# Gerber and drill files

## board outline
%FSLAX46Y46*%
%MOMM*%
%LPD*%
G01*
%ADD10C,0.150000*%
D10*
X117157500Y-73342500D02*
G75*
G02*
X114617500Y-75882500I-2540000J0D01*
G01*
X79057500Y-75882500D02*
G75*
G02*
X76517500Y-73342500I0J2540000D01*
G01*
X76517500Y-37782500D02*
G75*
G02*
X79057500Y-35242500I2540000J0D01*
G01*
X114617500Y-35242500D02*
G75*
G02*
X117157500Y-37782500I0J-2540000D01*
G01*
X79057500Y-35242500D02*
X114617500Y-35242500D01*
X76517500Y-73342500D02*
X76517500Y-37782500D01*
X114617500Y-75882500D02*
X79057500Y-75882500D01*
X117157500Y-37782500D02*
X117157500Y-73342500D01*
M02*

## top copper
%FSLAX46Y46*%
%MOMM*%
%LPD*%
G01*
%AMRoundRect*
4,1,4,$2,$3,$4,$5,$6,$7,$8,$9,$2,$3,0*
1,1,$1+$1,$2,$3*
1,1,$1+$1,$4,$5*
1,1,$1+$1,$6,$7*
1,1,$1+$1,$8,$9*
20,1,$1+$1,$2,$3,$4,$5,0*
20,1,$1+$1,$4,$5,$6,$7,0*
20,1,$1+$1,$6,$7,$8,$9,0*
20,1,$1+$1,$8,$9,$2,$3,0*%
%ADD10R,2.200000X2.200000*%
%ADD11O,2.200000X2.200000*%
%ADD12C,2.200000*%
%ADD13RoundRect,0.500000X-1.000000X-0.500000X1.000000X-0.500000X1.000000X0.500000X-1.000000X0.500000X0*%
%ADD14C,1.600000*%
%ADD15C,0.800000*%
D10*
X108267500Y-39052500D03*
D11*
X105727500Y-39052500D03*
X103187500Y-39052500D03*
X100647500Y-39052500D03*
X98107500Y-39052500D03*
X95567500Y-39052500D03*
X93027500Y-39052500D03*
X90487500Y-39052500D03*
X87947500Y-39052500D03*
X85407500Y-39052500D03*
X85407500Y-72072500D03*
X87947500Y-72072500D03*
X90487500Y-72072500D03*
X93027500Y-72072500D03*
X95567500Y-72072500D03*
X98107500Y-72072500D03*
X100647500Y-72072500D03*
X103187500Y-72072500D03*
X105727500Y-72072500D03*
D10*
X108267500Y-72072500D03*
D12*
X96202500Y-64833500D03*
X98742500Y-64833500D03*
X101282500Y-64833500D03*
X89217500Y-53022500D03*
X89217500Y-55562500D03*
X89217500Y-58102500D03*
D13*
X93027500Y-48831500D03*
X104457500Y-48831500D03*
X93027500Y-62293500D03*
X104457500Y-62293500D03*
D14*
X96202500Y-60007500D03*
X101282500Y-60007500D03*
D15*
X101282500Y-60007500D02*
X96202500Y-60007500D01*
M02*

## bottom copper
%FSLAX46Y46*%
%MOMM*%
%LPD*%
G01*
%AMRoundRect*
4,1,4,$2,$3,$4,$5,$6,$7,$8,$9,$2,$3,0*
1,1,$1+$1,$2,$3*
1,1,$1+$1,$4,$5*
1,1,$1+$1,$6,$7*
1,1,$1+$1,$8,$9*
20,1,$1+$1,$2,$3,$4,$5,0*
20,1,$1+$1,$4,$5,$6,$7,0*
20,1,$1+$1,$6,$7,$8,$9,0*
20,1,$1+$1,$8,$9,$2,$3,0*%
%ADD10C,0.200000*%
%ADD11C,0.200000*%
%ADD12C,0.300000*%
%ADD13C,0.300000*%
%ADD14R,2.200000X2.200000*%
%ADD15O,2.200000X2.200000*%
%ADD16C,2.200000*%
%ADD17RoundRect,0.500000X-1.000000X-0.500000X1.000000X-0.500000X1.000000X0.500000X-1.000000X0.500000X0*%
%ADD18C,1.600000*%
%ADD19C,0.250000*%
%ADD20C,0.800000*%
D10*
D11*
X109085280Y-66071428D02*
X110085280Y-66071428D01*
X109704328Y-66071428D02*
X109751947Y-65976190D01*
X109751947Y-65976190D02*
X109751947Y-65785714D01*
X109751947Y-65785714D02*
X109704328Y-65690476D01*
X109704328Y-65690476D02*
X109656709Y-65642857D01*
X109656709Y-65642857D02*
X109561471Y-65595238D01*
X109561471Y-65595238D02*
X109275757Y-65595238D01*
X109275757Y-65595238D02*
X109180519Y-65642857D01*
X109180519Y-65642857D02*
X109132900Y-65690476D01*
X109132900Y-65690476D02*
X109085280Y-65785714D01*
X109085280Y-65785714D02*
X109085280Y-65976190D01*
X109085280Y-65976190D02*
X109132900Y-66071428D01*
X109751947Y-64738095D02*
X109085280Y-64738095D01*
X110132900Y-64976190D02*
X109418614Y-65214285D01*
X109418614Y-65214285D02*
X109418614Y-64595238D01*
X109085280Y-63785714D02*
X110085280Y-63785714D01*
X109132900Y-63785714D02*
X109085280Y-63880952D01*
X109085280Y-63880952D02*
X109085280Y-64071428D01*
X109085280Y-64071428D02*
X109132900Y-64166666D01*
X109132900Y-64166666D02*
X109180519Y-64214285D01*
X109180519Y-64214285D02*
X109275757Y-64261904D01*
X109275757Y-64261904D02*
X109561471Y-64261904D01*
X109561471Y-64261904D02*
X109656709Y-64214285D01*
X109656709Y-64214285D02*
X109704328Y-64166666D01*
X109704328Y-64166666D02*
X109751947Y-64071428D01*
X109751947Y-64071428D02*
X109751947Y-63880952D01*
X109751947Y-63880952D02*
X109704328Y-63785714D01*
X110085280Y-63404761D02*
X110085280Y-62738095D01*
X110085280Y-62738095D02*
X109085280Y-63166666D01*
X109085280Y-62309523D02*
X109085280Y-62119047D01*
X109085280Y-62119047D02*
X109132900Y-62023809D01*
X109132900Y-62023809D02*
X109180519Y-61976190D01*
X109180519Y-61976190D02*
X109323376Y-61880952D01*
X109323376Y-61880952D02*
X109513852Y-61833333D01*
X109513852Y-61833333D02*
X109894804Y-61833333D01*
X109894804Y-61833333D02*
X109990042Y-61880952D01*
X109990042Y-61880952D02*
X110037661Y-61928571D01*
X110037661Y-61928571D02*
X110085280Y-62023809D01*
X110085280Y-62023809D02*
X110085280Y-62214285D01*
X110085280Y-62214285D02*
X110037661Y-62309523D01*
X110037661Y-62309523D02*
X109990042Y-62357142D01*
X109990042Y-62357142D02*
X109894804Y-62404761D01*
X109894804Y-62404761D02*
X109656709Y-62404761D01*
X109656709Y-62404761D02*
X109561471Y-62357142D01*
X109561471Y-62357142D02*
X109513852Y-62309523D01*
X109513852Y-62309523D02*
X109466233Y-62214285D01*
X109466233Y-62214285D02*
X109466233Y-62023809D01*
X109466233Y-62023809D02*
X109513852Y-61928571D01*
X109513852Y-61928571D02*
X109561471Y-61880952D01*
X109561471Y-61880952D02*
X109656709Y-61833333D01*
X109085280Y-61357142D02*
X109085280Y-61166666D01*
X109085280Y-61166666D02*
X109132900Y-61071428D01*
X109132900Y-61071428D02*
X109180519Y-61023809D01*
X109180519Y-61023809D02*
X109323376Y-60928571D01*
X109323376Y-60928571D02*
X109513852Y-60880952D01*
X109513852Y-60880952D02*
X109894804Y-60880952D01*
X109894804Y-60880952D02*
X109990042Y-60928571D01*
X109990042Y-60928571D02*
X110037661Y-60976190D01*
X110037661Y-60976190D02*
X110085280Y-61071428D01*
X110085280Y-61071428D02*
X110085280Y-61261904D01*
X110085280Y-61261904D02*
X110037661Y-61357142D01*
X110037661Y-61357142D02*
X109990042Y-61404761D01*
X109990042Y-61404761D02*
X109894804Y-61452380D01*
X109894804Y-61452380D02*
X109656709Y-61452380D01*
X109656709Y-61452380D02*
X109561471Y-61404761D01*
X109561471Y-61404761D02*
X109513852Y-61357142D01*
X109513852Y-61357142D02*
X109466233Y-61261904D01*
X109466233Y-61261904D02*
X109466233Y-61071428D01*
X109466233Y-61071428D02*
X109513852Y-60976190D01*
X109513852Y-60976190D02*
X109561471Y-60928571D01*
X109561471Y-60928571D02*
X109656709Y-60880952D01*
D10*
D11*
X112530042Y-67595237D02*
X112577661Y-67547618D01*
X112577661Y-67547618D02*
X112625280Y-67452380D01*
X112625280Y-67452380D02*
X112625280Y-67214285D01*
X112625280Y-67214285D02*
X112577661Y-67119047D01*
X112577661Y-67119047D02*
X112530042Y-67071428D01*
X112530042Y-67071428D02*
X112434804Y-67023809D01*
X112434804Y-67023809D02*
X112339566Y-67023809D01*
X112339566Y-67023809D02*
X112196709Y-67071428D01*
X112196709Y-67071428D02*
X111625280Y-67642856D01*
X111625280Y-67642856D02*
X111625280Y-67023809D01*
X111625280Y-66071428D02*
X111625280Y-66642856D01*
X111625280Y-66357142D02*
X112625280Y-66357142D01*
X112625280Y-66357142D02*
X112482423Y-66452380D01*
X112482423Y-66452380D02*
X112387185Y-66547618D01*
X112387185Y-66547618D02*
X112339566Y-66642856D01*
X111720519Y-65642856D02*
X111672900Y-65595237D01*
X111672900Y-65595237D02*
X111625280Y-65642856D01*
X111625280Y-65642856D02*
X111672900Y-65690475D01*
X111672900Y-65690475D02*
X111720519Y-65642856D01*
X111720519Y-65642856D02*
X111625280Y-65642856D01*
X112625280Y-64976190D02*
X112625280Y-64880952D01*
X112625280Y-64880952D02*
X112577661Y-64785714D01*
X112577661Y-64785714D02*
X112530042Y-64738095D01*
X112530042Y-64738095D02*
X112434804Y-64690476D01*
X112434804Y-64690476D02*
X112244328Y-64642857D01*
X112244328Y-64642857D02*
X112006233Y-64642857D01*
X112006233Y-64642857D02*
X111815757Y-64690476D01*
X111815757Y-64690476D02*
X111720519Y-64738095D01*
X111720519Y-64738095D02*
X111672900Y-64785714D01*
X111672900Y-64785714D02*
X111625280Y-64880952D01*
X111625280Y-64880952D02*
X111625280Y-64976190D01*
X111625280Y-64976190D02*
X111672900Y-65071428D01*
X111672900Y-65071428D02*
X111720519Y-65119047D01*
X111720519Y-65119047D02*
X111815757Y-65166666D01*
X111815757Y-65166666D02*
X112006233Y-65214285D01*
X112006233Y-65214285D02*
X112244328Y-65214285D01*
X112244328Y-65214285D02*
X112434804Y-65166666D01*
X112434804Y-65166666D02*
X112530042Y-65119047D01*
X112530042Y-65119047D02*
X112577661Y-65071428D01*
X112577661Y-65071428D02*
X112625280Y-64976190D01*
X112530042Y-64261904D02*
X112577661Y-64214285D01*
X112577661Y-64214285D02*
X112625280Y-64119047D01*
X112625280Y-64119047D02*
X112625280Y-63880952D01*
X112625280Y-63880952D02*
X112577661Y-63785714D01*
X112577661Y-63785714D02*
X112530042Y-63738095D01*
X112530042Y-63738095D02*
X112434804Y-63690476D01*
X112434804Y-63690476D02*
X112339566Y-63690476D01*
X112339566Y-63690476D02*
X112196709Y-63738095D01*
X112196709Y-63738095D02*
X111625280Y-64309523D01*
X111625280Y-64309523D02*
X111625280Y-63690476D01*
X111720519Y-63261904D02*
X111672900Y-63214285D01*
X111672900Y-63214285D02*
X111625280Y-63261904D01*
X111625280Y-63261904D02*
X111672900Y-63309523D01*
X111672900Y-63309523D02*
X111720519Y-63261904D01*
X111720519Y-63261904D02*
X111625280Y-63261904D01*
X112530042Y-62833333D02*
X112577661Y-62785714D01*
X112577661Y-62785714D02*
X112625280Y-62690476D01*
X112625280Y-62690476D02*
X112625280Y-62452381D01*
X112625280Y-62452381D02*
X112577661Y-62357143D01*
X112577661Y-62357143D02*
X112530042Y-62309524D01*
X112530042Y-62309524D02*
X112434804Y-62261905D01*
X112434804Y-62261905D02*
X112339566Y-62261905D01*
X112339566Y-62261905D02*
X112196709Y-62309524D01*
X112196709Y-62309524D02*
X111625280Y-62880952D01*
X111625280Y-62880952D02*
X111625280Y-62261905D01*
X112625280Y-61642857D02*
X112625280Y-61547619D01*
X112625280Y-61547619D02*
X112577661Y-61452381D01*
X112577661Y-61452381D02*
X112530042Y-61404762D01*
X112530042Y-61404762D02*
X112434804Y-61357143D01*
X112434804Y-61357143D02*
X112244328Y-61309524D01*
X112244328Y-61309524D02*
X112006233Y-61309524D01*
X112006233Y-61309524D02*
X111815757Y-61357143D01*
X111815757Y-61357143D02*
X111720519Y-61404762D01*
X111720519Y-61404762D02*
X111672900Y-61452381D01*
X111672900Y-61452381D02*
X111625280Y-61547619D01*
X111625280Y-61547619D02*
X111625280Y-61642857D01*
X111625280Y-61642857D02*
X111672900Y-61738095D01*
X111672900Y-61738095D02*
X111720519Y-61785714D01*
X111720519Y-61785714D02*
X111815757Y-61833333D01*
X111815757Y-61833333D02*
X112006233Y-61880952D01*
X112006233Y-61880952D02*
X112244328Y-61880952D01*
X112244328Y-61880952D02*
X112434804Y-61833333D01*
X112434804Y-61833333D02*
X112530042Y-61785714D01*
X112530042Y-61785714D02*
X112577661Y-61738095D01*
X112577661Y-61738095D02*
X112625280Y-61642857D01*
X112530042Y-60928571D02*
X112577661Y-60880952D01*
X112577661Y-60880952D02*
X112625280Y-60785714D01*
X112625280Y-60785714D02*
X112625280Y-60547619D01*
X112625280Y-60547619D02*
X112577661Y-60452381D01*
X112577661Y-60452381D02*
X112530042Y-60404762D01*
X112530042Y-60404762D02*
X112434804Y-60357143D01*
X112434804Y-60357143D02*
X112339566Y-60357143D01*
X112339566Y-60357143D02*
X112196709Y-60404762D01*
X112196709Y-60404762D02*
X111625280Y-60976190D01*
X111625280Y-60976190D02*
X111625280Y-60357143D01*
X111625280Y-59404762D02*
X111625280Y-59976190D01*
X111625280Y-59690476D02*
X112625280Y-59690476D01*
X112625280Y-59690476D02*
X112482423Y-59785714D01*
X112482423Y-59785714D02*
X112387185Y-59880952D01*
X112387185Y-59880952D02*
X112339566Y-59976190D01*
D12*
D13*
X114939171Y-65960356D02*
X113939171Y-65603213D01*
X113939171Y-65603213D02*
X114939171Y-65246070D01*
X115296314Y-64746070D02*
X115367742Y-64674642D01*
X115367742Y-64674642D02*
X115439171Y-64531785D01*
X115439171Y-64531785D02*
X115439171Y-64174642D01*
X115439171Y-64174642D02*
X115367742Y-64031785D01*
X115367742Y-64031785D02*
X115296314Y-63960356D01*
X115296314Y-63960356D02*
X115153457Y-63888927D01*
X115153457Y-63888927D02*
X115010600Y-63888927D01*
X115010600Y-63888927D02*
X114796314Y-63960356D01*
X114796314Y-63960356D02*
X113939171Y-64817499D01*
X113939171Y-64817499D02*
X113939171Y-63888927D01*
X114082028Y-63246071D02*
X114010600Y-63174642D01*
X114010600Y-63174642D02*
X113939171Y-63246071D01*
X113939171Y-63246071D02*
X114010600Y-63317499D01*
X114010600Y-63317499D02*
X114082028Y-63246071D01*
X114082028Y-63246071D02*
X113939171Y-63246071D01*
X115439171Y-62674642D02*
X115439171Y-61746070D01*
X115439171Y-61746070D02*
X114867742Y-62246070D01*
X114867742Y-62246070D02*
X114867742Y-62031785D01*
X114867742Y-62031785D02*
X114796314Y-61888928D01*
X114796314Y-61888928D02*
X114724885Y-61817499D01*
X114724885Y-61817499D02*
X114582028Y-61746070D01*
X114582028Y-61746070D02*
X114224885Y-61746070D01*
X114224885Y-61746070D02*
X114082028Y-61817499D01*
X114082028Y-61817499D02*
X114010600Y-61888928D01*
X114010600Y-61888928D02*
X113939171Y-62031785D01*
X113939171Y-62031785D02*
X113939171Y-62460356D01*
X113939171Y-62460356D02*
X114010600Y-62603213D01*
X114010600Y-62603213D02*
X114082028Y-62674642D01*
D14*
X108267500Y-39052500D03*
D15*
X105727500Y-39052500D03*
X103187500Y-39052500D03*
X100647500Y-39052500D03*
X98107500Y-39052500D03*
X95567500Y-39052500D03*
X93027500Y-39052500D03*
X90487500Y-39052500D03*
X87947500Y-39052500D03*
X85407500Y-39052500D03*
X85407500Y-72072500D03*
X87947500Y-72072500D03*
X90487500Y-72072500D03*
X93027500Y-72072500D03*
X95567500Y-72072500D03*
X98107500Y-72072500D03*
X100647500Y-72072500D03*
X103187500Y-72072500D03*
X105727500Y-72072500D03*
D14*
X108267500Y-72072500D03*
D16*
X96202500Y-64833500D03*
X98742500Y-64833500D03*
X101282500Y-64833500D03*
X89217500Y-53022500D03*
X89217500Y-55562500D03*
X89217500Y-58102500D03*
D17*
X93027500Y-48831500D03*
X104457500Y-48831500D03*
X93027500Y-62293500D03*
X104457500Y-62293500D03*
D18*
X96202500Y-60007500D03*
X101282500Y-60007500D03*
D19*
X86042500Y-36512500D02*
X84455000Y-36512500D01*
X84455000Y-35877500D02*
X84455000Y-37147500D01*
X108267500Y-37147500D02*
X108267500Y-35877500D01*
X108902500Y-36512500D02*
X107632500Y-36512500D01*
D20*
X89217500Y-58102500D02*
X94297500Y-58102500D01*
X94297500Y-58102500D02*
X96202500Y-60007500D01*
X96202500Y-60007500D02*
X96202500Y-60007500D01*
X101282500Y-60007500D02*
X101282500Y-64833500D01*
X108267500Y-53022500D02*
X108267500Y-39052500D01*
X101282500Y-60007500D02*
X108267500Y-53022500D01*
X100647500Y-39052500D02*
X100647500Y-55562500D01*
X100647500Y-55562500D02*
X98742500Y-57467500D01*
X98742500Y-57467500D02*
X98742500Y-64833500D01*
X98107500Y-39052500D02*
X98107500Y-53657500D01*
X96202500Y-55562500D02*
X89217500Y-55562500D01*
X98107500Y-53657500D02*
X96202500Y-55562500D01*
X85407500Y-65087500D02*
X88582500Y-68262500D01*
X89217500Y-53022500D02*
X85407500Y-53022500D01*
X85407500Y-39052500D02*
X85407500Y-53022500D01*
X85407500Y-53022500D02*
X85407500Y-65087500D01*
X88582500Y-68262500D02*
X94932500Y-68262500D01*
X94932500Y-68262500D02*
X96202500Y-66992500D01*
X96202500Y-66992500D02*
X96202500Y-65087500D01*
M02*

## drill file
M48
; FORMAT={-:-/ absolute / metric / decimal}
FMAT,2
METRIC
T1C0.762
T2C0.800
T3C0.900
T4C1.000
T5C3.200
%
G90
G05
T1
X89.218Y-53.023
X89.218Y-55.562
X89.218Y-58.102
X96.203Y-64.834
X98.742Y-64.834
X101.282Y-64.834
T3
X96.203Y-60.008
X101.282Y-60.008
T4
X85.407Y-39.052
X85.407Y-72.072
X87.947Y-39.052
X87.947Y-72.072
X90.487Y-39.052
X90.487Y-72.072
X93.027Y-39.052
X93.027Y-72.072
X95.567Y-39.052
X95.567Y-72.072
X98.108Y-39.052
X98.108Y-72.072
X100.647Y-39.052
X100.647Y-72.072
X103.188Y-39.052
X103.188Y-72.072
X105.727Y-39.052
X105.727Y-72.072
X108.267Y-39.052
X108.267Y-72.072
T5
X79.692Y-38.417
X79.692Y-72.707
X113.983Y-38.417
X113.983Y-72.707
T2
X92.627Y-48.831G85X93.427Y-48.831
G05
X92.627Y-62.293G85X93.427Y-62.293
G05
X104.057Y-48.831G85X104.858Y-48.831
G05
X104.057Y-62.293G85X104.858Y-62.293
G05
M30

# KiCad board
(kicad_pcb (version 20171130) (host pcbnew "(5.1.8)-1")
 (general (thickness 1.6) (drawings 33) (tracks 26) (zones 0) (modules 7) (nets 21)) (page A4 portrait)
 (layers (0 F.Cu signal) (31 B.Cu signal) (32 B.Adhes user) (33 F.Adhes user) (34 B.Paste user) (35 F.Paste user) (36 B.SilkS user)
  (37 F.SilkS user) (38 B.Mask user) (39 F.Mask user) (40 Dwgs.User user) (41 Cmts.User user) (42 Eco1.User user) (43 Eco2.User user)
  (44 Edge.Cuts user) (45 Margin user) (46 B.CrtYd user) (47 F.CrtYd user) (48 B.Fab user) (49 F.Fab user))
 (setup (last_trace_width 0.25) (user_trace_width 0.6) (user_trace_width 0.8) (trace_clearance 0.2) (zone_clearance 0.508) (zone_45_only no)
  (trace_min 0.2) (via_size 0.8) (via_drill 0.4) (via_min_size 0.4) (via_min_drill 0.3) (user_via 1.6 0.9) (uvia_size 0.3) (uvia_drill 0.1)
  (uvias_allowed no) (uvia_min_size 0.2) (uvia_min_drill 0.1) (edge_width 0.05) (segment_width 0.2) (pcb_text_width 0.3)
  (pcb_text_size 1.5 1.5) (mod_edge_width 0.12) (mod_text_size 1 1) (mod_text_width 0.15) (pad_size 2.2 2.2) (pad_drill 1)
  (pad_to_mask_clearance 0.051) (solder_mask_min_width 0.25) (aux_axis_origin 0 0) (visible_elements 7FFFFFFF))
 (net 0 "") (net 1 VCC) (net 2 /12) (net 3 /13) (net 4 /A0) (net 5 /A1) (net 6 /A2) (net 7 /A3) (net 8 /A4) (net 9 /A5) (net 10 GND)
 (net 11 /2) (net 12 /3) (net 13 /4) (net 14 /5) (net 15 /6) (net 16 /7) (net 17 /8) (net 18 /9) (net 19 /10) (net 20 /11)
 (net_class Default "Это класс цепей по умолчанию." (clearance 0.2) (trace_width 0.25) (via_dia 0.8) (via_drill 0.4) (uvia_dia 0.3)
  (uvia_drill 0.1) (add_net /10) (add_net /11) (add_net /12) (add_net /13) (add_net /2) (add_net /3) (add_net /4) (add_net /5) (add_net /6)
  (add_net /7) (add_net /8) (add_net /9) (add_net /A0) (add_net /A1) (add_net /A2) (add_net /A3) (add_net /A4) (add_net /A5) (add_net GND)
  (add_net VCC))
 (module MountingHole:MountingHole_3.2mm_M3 (layer F.Cu) (at 113.9825 38.4175 270)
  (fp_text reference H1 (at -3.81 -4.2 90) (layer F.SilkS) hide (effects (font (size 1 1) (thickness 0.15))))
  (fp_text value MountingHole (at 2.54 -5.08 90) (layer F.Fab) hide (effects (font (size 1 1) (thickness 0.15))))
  (pad 1 np_thru_hole circle (at 0 0 270) (size 3.2 3.2) (drill 3.2) (layers *.Cu *.Mask)))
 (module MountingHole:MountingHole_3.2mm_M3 (layer F.Cu) (at 79.6925 38.4175 270)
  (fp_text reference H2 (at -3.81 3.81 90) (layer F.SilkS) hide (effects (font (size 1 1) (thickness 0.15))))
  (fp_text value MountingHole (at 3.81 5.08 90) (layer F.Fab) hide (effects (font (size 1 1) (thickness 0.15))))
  (pad 1 np_thru_hole circle (at 0 0 270) (size 3.2 3.2) (drill 3.2) (layers *.Cu *.Mask)))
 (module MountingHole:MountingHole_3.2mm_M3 (layer F.Cu) (at 113.9825 72.7075 270)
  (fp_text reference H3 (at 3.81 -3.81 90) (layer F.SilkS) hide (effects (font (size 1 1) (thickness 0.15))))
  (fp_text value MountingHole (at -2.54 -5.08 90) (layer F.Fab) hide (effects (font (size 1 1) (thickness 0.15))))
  (pad 1 np_thru_hole circle (at 0 0 270) (size 3.2 3.2) (drill 3.2) (layers *.Cu *.Mask)))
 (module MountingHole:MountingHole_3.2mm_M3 (layer F.Cu) (at 79.6925 72.7075 270)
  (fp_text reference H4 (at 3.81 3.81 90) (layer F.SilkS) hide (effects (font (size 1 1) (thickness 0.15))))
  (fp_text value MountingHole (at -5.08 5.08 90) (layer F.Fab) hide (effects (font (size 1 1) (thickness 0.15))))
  (pad 1 np_thru_hole circle (at 0 0 270) (size 3.2 3.2) (drill 3.2) (layers *.Cu *.Mask)))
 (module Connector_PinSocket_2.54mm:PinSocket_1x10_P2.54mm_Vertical (layer F.Cu) (at 108.2675 39.0525 270)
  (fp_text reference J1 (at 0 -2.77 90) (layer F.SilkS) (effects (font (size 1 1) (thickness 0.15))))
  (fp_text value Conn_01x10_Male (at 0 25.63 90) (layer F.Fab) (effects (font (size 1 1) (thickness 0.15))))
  (pad 1 thru_hole rect (at 0 0 270) (size 2.2 2.2) (drill 1) (layers *.Cu *.Mask) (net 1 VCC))
  (pad 2 thru_hole oval (at 0 2.54 270) (size 2.2 2.2) (drill 1) (layers *.Cu *.Mask) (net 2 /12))
  (pad 3 thru_hole oval (at 0 5.08 270) (size 2.2 2.2) (drill 1) (layers *.Cu *.Mask) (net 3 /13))
  (pad 4 thru_hole oval (at 0 7.62 270) (size 2.2 2.2) (drill 1) (layers *.Cu *.Mask) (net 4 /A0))
  (pad 5 thru_hole oval (at 0 10.16 270) (size 2.2 2.2) (drill 1) (layers *.Cu *.Mask) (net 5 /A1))
  (pad 6 thru_hole oval (at 0 12.7 270) (size 2.2 2.2) (drill 1) (layers *.Cu *.Mask) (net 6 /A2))
  (pad 7 thru_hole oval (at 0 15.24 270) (size 2.2 2.2) (drill 1) (layers *.Cu *.Mask) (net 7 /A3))
  (pad 8 thru_hole oval (at 0 17.78 270) (size 2.2 2.2) (drill 1) (layers *.Cu *.Mask) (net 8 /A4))
  (pad 9 thru_hole oval (at 0 20.32 270) (size 2.2 2.2) (drill 1) (layers *.Cu *.Mask) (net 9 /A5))
  (pad 10 thru_hole oval (at 0 22.86 270) (size 2.2 2.2) (drill 1) (layers *.Cu *.Mask) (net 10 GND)))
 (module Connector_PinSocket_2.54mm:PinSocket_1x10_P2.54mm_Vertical (layer F.Cu) (at 108.2675 72.0725 270)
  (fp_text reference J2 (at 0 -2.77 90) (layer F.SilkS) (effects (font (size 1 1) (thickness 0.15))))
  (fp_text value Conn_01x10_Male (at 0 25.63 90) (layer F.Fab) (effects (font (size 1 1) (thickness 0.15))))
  (pad 10 thru_hole oval (at 0 22.86 270) (size 2.2 2.2) (drill 1) (layers *.Cu *.Mask) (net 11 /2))
  (pad 9 thru_hole oval (at 0 20.32 270) (size 2.2 2.2) (drill 1) (layers *.Cu *.Mask) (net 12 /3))
  (pad 8 thru_hole oval (at 0 17.78 270) (size 2.2 2.2) (drill 1) (layers *.Cu *.Mask) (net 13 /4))
  (pad 7 thru_hole oval (at 0 15.24 270) (size 2.2 2.2) (drill 1) (layers *.Cu *.Mask) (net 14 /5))
  (pad 6 thru_hole oval (at 0 12.7 270) (size 2.2 2.2) (drill 1) (layers *.Cu *.Mask) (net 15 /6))
  (pad 5 thru_hole oval (at 0 10.16 270) (size 2.2 2.2) (drill 1) (layers *.Cu *.Mask) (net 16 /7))
  (pad 4 thru_hole oval (at 0 7.62 270) (size 2.2 2.2) (drill 1) (layers *.Cu *.Mask) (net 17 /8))
  (pad 3 thru_hole oval (at 0 5.08 270) (size 2.2 2.2) (drill 1) (layers *.Cu *.Mask) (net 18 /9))
  (pad 2 thru_hole oval (at 0 2.54 270) (size 2.2 2.2) (drill 1) (layers *.Cu *.Mask) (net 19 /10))
  (pad 1 thru_hole rect (at 0 0 270) (size 2.2 2.2) (drill 1) (layers *.Cu *.Mask) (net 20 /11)))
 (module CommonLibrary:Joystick (layer F.Cu) (at 98.7425 55.3085)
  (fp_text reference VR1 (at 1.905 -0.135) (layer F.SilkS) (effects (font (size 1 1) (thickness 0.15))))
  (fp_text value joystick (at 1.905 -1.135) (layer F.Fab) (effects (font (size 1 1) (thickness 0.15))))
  (pad 3 thru_hole circle (at -2.54 9.525) (size 2.2 2.2) (drill 0.762) (layers *.Cu *.Mask) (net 10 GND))
  (pad 2 thru_hole circle (at 0 9.525) (size 2.2 2.2) (drill 0.762) (layers *.Cu *.Mask) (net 4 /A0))
  (pad 1 thru_hole circle (at 2.54 9.525) (size 2.2 2.2) (drill 0.762) (layers *.Cu *.Mask) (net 1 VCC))
  (pad 4 thru_hole circle (at -9.525 -2.286) (size 2.2 2.2) (drill 0.762) (layers *.Cu *.Mask) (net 10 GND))
  (pad 5 thru_hole circle (at -9.525 0.254) (size 2.2 2.2) (drill 0.762) (layers *.Cu *.Mask) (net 5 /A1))
  (pad 6 thru_hole circle (at -9.525 2.794) (size 2.2 2.2) (drill 0.762) (layers *.Cu *.Mask) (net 1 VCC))
  (pad "" thru_hole roundrect (at -5.715 -6.477) (size 3 2) (drill oval 1.6 0.8) (layers *.Cu *.Mask) (roundrect_rratio 0.25))
  (pad "" thru_hole roundrect (at 5.715 -6.477) (size 3 2) (drill oval 1.6 0.8) (layers *.Cu *.Mask) (roundrect_rratio 0.25))
  (pad "" thru_hole roundrect (at -5.715 6.985) (size 3 2) (drill oval 1.6 0.8) (layers *.Cu *.Mask) (roundrect_rratio 0.25))
  (pad "" thru_hole roundrect (at 5.715 6.985) (size 3 2) (drill oval 1.6 0.8) (layers *.Cu *.Mask) (roundrect_rratio 0.25)))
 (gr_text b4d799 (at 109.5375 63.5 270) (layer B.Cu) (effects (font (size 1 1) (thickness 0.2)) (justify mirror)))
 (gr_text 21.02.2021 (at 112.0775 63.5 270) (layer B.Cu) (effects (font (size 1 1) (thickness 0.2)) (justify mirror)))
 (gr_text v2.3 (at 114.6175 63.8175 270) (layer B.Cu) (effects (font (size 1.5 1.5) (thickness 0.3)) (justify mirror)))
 (gr_arc (start 114.6175 73.3425) (end 114.6175 75.8825) (angle -90) (layer Edge.Cuts) (width 0.15))
 (gr_arc (start 79.0575 73.3425) (end 76.5175 73.3425) (angle -90) (layer Edge.Cuts) (width 0.15))
 (gr_arc (start 79.0575 37.7825) (end 79.0575 35.2425) (angle -90) (layer Edge.Cuts) (width 0.15))
 (gr_arc (start 114.6175 37.7825) (end 117.1575 37.7825) (angle -90) (layer Edge.Cuts) (width 0.15))
 (gr_line (start 79.0575 35.2425) (end 114.6175 35.2425) (layer Edge.Cuts) (width 0.15))
 (gr_line (start 76.5175 73.3425) (end 76.5175 37.7825) (layer Edge.Cuts) (width 0.15))
 (gr_line (start 114.6175 75.8825) (end 79.0575 75.8825) (layer Edge.Cuts) (width 0.15))
 (gr_line (start 117.1575 37.7825) (end 117.1575 73.3425) (layer Edge.Cuts) (width 0.15))
 (segment (start 86.0425 36.5125) (end 84.455 36.5125) (width 0.25) (layer B.Cu) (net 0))
 (segment (start 84.455 35.8775) (end 84.455 37.1475) (width 0.25) (layer B.Cu) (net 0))
 (segment (start 108.2675 37.1475) (end 108.2675 35.8775) (width 0.25) (layer B.Cu) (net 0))
 (segment (start 108.9025 36.5125) (end 107.6325 36.5125) (width 0.25) (layer B.Cu) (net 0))
 (segment (start 89.2175 58.1025) (end 94.2975 58.1025) (width 0.8) (layer B.Cu) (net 1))
 (segment (start 94.2975 58.1025) (end 96.2025 60.0075) (width 0.8) (layer B.Cu) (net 1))
 (segment (start 96.2025 60.0075) (end 96.2025 60.0075) (width 0.8) (layer B.Cu) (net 1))
 (via (at 96.2025 60.0075) (size 1.6) (drill 0.9) (layers F.Cu B.Cu) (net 1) (status 1000000))
 (via (at 101.2825 60.0075) (size 1.6) (drill 0.9) (layers F.Cu B.Cu) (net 1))
 (segment (start 101.2825 60.0075) (end 101.2825 64.8335) (width 0.8) (layer B.Cu) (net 1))
 (segment (start 108.2675 53.0225) (end 108.2675 39.0525) (width 0.8) (layer B.Cu) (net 1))
 (segment (start 101.2825 60.0075) (end 108.2675 53.0225) (width 0.8) (layer B.Cu) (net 1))
 (segment (start 101.2825 60.0075) (end 96.2025 60.0075) (width 0.8) (layer F.Cu) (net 1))
 (segment (start 100.6475 39.0525) (end 100.6475 55.5625) (width 0.8) (layer B.Cu) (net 4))
 (segment (start 100.6475 55.5625) (end 98.7425 57.4675) (width 0.8) (layer B.Cu) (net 4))
 (segment (start 98.7425 57.4675) (end 98.7425 64.8335) (width 0.8) (layer B.Cu) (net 4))
 (segment (start 98.1075 39.0525) (end 98.1075 53.6575) (width 0.8) (layer B.Cu) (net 5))
 (segment (start 96.2025 55.5625) (end 89.2175 55.5625) (width 0.8) (layer B.Cu) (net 5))
 (segment (start 98.1075 53.6575) (end 96.2025 55.5625) (width 0.8) (layer B.Cu) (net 5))
 (segment (start 85.4075 65.0875) (end 88.5825 68.2625) (width 0.8) (layer B.Cu) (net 10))
 (segment (start 89.2175 53.0225) (end 85.4075 53.0225) (width 0.8) (layer B.Cu) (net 10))
 (segment (start 85.4075 39.0525) (end 85.4075 53.0225) (width 0.8) (layer B.Cu) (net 10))
 (segment (start 85.4075 53.0225) (end 85.4075 65.0875) (width 0.8) (layer B.Cu) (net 10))
 (segment (start 88.5825 68.2625) (end 94.9325 68.2625) (width 0.8) (layer B.Cu) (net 10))
 (segment (start 94.9325 68.2625) (end 96.2025 66.9925) (width 0.8) (layer B.Cu) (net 10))
 (segment (start 96.2025 66.9925) (end 96.2025 65.0875) (width 0.8) (layer B.Cu) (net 10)))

